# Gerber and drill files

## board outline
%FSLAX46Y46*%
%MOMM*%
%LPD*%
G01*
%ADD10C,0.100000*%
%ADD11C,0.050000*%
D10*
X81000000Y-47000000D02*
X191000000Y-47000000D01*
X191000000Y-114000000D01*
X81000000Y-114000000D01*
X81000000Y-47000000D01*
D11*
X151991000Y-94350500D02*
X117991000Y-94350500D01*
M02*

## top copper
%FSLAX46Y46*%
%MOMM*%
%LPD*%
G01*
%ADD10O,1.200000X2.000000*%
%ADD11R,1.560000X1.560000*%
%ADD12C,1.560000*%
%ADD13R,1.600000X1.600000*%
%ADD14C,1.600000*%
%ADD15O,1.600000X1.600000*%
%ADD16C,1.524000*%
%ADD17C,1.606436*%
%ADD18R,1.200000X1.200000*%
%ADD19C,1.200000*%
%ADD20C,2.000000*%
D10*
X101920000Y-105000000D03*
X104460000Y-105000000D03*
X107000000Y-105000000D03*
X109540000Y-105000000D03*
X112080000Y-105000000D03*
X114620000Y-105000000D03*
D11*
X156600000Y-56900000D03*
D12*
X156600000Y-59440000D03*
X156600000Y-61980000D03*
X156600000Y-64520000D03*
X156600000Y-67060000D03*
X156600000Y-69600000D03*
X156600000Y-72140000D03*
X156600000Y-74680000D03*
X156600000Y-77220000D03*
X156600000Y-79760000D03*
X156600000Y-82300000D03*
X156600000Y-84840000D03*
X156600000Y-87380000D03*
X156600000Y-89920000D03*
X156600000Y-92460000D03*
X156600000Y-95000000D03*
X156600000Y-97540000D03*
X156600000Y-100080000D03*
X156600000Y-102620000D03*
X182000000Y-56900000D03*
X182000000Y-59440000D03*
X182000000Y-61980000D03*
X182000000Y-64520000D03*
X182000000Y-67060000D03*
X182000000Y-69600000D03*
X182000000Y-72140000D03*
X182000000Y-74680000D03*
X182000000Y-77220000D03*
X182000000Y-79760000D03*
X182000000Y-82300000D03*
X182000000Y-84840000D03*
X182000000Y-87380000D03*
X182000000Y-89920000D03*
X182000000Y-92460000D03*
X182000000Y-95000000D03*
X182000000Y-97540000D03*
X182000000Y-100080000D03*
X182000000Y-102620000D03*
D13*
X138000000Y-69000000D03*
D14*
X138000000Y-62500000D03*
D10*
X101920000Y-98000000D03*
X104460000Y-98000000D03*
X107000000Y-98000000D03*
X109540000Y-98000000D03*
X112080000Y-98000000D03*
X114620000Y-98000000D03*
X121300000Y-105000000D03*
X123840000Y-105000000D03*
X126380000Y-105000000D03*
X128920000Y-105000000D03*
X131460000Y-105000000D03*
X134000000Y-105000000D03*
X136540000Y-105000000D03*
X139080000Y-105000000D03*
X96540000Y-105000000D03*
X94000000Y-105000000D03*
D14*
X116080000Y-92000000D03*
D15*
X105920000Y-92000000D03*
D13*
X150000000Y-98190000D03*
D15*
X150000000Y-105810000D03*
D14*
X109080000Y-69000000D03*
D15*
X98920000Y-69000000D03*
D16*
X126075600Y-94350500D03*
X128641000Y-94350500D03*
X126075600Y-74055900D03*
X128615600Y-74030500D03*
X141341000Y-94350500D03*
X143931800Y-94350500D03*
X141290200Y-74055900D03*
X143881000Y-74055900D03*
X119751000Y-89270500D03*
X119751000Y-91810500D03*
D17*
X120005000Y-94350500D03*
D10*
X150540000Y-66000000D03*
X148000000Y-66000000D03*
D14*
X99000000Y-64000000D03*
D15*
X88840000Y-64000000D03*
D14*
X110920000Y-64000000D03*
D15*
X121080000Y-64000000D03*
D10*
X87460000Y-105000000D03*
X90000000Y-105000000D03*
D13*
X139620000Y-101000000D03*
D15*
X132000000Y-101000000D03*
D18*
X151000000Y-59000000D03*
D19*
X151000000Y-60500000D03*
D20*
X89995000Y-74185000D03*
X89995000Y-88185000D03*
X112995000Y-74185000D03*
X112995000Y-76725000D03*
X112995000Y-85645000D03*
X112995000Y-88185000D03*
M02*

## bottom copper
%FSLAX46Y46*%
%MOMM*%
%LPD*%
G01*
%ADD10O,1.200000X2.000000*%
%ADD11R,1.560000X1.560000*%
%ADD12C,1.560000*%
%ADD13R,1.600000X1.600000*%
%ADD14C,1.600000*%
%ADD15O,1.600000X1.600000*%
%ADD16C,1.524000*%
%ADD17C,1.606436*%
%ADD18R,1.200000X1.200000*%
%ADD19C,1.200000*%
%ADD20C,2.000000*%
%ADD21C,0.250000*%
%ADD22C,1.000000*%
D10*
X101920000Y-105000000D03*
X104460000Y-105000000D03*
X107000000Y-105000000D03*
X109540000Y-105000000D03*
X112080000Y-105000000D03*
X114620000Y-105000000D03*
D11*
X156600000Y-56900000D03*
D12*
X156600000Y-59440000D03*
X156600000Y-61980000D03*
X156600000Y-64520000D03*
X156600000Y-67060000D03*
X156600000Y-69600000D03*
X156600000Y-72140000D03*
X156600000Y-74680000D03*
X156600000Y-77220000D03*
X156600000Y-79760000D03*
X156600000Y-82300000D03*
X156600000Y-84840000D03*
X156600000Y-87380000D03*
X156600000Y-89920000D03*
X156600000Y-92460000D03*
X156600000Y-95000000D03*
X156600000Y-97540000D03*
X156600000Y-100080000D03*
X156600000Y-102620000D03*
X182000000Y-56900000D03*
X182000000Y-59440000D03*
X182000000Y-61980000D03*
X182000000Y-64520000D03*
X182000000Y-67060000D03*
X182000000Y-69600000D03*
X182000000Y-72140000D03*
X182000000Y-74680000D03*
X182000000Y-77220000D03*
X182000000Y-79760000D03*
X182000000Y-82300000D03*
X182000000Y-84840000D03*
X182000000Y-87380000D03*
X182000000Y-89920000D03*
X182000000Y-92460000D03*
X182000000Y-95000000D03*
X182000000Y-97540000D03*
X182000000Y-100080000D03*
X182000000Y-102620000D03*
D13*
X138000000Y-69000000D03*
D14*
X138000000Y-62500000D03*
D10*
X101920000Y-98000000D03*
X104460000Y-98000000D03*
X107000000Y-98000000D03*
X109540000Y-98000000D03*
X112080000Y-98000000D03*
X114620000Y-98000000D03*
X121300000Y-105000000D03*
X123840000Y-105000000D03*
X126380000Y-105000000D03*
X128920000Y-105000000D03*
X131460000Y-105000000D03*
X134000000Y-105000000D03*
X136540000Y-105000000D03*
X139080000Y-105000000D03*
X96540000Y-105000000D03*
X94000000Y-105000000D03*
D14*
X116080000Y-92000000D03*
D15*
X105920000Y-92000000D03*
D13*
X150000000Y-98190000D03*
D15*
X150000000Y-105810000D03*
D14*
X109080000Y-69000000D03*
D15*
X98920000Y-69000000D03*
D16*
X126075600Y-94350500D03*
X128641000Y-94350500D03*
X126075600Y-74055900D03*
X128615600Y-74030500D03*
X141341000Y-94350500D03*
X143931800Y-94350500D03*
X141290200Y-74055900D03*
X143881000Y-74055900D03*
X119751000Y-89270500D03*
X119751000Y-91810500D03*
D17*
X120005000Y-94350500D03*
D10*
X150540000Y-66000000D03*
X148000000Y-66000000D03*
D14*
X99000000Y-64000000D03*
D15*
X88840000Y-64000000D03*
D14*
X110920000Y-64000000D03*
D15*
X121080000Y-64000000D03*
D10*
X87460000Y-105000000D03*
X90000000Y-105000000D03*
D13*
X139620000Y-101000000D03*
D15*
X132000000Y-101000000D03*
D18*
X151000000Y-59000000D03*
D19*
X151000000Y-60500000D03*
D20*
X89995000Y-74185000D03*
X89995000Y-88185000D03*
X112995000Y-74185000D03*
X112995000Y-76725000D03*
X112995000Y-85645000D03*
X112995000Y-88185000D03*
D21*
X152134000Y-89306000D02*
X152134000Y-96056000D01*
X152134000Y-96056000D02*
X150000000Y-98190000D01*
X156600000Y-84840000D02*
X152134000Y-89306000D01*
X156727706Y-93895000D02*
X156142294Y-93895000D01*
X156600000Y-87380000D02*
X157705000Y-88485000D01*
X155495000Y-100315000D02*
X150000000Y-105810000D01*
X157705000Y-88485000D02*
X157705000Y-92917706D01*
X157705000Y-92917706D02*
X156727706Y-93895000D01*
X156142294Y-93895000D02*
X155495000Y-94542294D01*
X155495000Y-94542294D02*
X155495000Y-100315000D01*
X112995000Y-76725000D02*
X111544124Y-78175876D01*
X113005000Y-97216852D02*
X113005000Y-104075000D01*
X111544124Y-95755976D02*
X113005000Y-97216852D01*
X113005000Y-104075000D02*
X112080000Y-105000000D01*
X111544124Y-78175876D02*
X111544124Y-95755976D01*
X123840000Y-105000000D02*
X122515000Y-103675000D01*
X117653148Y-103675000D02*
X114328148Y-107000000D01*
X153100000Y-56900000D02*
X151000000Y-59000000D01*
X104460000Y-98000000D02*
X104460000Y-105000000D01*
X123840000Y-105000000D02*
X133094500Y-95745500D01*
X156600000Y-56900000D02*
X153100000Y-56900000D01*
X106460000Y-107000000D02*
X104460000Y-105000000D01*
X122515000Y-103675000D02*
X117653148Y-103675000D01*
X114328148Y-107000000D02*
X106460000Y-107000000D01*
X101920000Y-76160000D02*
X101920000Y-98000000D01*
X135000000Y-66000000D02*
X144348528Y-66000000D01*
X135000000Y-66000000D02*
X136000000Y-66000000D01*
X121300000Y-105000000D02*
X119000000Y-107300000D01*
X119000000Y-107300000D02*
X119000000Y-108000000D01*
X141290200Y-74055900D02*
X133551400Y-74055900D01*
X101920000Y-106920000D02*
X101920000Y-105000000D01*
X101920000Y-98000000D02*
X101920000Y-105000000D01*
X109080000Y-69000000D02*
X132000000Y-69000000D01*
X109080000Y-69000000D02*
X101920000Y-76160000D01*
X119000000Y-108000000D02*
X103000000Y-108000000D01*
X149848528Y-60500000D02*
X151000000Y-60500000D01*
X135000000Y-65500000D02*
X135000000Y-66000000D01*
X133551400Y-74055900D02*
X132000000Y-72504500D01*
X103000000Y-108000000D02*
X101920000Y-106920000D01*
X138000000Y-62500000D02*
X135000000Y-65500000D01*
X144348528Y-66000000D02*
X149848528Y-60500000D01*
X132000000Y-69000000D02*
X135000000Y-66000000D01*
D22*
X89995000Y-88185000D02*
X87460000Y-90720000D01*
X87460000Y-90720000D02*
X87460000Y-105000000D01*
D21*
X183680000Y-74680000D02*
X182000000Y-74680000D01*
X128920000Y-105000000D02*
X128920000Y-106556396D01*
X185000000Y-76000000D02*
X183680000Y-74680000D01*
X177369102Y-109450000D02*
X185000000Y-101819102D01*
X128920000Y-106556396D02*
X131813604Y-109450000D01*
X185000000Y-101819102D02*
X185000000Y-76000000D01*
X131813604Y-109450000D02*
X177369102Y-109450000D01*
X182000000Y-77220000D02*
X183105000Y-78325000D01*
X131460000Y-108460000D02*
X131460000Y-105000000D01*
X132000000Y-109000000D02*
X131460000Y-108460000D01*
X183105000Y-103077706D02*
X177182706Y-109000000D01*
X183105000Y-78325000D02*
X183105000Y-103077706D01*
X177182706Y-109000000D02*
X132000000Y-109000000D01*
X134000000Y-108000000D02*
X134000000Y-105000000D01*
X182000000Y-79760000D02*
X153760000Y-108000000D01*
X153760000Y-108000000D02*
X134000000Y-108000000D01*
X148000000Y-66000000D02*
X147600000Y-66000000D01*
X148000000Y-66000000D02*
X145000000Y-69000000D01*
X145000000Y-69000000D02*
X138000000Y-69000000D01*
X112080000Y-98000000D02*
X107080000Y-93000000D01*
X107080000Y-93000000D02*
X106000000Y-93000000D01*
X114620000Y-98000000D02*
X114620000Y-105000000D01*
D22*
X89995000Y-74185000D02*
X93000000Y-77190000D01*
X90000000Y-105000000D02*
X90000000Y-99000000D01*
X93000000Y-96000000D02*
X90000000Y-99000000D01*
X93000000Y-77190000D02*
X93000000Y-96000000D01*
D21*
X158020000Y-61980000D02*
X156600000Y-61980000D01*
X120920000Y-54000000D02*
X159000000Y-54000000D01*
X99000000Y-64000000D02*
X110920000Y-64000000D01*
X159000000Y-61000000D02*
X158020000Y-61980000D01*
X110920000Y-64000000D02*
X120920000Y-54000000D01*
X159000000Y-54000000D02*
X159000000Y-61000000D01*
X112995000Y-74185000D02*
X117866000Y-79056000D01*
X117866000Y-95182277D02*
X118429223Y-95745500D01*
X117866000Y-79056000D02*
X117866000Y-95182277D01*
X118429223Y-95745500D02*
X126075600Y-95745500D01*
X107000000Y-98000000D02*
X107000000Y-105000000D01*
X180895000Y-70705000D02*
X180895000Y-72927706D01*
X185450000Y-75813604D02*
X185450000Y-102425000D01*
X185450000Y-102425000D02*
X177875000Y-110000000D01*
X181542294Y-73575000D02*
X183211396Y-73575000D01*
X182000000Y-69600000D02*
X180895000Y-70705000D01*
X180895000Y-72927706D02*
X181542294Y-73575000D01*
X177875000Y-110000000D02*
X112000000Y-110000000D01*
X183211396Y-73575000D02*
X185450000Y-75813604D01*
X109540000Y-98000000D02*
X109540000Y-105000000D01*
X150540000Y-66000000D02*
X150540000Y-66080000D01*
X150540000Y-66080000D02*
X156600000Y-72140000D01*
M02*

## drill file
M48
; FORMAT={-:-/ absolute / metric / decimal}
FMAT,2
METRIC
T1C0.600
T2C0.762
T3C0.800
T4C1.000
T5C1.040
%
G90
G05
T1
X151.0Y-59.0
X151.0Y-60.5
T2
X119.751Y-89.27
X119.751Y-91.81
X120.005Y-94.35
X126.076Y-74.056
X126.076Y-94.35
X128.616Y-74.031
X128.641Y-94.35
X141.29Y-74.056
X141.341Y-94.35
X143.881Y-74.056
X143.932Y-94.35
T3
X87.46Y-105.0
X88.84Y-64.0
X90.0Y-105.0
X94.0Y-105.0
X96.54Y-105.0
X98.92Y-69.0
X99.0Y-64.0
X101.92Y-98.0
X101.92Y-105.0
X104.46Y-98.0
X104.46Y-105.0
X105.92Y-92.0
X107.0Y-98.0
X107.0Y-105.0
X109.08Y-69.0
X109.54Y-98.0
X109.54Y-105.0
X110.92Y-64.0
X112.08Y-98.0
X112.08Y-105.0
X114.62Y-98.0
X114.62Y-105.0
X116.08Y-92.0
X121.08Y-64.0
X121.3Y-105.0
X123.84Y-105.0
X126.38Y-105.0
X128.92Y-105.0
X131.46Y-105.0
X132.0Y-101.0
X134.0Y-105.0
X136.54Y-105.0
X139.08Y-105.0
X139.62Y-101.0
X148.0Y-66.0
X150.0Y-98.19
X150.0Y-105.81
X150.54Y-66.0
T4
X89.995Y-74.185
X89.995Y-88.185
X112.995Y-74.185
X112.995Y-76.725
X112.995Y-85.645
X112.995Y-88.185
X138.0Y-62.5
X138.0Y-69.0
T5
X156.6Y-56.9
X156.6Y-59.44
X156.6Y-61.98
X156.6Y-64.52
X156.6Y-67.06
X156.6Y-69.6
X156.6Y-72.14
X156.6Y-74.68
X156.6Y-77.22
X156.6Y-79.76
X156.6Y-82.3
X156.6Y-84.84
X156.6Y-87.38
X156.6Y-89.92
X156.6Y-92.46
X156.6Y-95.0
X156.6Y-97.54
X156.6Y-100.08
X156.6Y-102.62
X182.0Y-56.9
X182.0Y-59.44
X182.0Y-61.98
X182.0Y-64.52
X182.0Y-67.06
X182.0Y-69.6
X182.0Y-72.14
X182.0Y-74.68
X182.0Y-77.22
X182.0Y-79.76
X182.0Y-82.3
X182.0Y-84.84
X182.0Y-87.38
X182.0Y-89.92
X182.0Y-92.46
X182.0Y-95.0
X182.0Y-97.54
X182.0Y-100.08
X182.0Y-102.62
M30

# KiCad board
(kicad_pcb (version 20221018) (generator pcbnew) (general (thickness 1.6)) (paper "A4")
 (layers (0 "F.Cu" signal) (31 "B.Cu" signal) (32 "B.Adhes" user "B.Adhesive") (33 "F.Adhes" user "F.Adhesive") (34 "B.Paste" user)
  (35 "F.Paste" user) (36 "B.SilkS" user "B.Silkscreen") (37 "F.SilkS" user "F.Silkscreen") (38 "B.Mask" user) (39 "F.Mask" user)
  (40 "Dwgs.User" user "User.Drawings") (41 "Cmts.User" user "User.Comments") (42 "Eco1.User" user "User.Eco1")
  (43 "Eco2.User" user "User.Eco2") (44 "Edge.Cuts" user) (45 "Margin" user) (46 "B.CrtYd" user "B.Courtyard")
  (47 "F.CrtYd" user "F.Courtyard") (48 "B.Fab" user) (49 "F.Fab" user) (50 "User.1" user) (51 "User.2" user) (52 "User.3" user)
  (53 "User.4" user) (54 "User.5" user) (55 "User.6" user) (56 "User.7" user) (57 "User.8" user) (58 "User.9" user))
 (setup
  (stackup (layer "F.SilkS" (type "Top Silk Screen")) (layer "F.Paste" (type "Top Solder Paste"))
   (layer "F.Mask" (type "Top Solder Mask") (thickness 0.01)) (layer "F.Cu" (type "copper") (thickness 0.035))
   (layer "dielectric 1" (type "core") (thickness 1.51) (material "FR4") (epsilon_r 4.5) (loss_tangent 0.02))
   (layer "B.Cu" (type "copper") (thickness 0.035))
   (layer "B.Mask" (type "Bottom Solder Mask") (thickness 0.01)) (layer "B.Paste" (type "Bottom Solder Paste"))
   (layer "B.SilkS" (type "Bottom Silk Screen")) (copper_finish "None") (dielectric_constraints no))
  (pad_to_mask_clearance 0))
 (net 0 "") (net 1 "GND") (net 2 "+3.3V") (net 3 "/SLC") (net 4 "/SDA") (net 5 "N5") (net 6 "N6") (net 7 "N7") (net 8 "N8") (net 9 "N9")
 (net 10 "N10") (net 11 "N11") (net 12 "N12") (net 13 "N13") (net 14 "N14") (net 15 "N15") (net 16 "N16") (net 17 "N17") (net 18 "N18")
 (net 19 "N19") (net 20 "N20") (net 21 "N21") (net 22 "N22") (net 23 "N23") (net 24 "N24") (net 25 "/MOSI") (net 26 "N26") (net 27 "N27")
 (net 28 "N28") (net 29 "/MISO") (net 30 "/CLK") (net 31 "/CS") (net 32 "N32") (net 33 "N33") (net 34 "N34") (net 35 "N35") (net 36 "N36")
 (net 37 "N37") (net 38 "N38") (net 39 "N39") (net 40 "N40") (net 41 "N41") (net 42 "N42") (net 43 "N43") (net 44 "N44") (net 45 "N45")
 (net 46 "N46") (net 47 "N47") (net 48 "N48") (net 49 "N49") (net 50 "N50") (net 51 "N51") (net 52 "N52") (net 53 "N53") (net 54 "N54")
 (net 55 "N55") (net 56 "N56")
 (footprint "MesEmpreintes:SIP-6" (layer "F.Cu") (at 108.27 105)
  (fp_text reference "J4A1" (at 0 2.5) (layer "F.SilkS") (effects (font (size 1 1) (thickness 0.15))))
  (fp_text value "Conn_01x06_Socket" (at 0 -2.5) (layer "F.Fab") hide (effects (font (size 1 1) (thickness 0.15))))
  (pad "1" thru_hole oval (at -6.35 0) (size 1.2 2) (drill 0.8) (layers "*.Cu" "*.Mask") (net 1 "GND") (thermal_bridge_angle 45))
  (pad "2" thru_hole oval (at -3.81 0) (size 1.2 2) (drill 0.8) (layers "*.Cu" "*.Mask") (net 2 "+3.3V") (thermal_bridge_angle 45))
  (pad "3" thru_hole oval (at -1.27 0) (size 1.2 2) (drill 0.8) (layers "*.Cu" "*.Mask") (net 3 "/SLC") (thermal_bridge_angle 45))
  (pad "4" thru_hole oval (at 1.27 0) (size 1.2 2) (drill 0.8) (layers "*.Cu" "*.Mask") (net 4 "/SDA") (thermal_bridge_angle 45))
  (pad "5" thru_hole oval (at 3.81 0) (size 1.2 2) (drill 0.8) (layers "*.Cu" "*.Mask") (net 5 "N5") (thermal_bridge_angle 45))
  (pad "6" thru_hole oval (at 6.35 0) (size 1.2 2) (drill 0.8) (layers "*.Cu" "*.Mask") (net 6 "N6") (thermal_bridge_angle 45)))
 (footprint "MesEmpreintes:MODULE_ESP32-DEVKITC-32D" (layer "F.Cu") (at 169.3 75.97)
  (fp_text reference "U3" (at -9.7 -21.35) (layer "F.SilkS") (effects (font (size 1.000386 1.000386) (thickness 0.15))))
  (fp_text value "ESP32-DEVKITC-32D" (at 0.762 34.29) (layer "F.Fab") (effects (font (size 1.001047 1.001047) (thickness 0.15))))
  (pad "J2-1" thru_hole rect (at -12.7 -19.07) (size 1.56 1.56) (drill 1.04) (layers "*.Cu" "*.Mask") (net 2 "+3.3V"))
  (pad "J2-2" thru_hole circle (at -12.7 -16.53) (size 1.56 1.56) (drill 1.04) (layers "*.Cu" "*.Mask") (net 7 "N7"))
  (pad "J2-3" thru_hole circle (at -12.7 -13.99) (size 1.56 1.56) (drill 1.04) (layers "*.Cu" "*.Mask") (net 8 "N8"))
  (pad "J2-4" thru_hole circle (at -12.7 -11.45) (size 1.56 1.56) (drill 1.04) (layers "*.Cu" "*.Mask") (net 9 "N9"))
  (pad "J2-5" thru_hole circle (at -12.7 -8.91) (size 1.56 1.56) (drill 1.04) (layers "*.Cu" "*.Mask") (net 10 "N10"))
  (pad "J2-6" thru_hole circle (at -12.7 -6.37) (size 1.56 1.56) (drill 1.04) (layers "*.Cu" "*.Mask") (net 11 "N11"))
  (pad "J2-7" thru_hole circle (at -12.7 -3.83) (size 1.56 1.56) (drill 1.04) (layers "*.Cu" "*.Mask") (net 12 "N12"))
  (pad "J2-8" thru_hole circle (at -12.7 -1.29) (size 1.56 1.56) (drill 1.04) (layers "*.Cu" "*.Mask") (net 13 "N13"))
  (pad "J2-9" thru_hole circle (at -12.7 1.25) (size 1.56 1.56) (drill 1.04) (layers "*.Cu" "*.Mask") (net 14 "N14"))
  (pad "J2-10" thru_hole circle (at -12.7 3.79) (size 1.56 1.56) (drill 1.04) (layers "*.Cu" "*.Mask") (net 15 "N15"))
  (pad "J2-11" thru_hole circle (at -12.7 6.33) (size 1.56 1.56) (drill 1.04) (layers "*.Cu" "*.Mask") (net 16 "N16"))
  (pad "J2-12" thru_hole circle (at -12.7 8.87) (size 1.56 1.56) (drill 1.04) (layers "*.Cu" "*.Mask") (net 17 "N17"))
  (pad "J2-13" thru_hole circle (at -12.7 11.41) (size 1.56 1.56) (drill 1.04) (layers "*.Cu" "*.Mask") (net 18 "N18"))
  (pad "J2-14" thru_hole circle (at -12.7 13.95) (size 1.56 1.56) (drill 1.04) (layers "*.Cu" "*.Mask") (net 1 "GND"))
  (pad "J2-15" thru_hole circle (at -12.7 16.49) (size 1.56 1.56) (drill 1.04) (layers "*.Cu" "*.Mask") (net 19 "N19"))
  (pad "J2-16" thru_hole circle (at -12.7 19.03) (size 1.56 1.56) (drill 1.04) (layers "*.Cu" "*.Mask") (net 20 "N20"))
  (pad "J2-17" thru_hole circle (at -12.7 21.57) (size 1.56 1.56) (drill 1.04) (layers "*.Cu" "*.Mask") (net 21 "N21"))
  (pad "J2-18" thru_hole circle (at -12.7 24.11) (size 1.56 1.56) (drill 1.04) (layers "*.Cu" "*.Mask") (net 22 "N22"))
  (pad "J2-19" thru_hole circle (at -12.7 26.65) (size 1.56 1.56) (drill 1.04) (layers "*.Cu" "*.Mask") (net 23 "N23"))
  (pad "J3-1" thru_hole circle (at 12.7 -19.07) (size 1.56 1.56) (drill 1.04) (layers "*.Cu" "*.Mask") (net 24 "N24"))
  (pad "J3-2" thru_hole circle (at 12.7 -16.53) (size 1.56 1.56) (drill 1.04) (layers "*.Cu" "*.Mask") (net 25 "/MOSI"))
  (pad "J3-3" thru_hole circle (at 12.7 -13.99) (size 1.56 1.56) (drill 1.04) (layers "*.Cu" "*.Mask") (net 3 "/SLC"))
  (pad "J3-4" thru_hole circle (at 12.7 -11.45) (size 1.56 1.56) (drill 1.04) (layers "*.Cu" "*.Mask") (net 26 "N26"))
  (pad "J3-5" thru_hole circle (at 12.7 -8.91) (size 1.56 1.56) (drill 1.04) (layers "*.Cu" "*.Mask") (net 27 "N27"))
  (pad "J3-6" thru_hole circle (at 12.7 -6.37) (size 1.56 1.56) (drill 1.04) (layers "*.Cu" "*.Mask") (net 4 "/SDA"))
  (pad "J3-7" thru_hole circle (at 12.7 -3.83) (size 1.56 1.56) (drill 1.04) (layers "*.Cu" "*.Mask") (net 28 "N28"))
  (pad "J3-8" thru_hole circle (at 12.7 -1.29) (size 1.56 1.56) (drill 1.04) (layers "*.Cu" "*.Mask") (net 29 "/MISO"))
  (pad "J3-9" thru_hole circle (at 12.7 1.25) (size 1.56 1.56) (drill 1.04) (layers "*.Cu" "*.Mask") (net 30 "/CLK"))
  (pad "J3-10" thru_hole circle (at 12.7 3.79) (size 1.56 1.56) (drill 1.04) (layers "*.Cu" "*.Mask") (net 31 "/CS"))
  (pad "J3-11" thru_hole circle (at 12.7 6.33) (size 1.56 1.56) (drill 1.04) (layers "*.Cu" "*.Mask") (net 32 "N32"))
  (pad "J3-12" thru_hole circle (at 12.7 8.87) (size 1.56 1.56) (drill 1.04) (layers "*.Cu" "*.Mask") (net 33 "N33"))
  (pad "J3-13" thru_hole circle (at 12.7 11.41) (size 1.56 1.56) (drill 1.04) (layers "*.Cu" "*.Mask") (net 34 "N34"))
  (pad "J3-14" thru_hole circle (at 12.7 13.95) (size 1.56 1.56) (drill 1.04) (layers "*.Cu" "*.Mask") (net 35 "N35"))
  (pad "J3-15" thru_hole circle (at 12.7 16.49) (size 1.56 1.56) (drill 1.04) (layers "*.Cu" "*.Mask") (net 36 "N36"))
  (pad "J3-16" thru_hole circle (at 12.7 19.03) (size 1.56 1.56) (drill 1.04) (layers "*.Cu" "*.Mask") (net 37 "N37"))
  (pad "J3-17" thru_hole circle (at 12.7 21.57) (size 1.56 1.56) (drill 1.04) (layers "*.Cu" "*.Mask") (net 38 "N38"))
  (pad "J3-18" thru_hole circle (at 12.7 24.11) (size 1.56 1.56) (drill 1.04) (layers "*.Cu" "*.Mask") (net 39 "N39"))
  (pad "J3-19" thru_hole circle (at 12.7 26.65) (size 1.56 1.56) (drill 1.04) (layers "*.Cu" "*.Mask") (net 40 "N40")))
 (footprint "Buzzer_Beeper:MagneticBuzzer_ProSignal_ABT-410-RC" (layer "F.Cu") (at 138 69 90)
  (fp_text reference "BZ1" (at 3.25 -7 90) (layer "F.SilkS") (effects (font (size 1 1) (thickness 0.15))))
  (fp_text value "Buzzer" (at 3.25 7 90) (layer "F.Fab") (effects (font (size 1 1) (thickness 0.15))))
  (pad "1" thru_hole rect (at 0 0 90) (size 1.6 1.6) (drill 1) (layers "*.Cu" "*.Mask") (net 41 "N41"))
  (pad "2" thru_hole circle (at 6.5 0 90) (size 1.6 1.6) (drill 1) (layers "*.Cu" "*.Mask") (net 1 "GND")))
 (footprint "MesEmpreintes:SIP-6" (layer "F.Cu") (at 108.27 98)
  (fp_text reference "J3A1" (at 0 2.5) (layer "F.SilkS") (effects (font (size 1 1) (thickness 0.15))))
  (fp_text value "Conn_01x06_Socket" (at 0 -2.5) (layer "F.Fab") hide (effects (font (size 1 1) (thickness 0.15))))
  (pad "1" thru_hole oval (at -6.35 0) (size 1.2 2) (drill 0.8) (layers "*.Cu" "*.Mask") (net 1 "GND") (thermal_bridge_angle 45))
  (pad "2" thru_hole oval (at -3.81 0) (size 1.2 2) (drill 0.8) (layers "*.Cu" "*.Mask") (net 2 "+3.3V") (thermal_bridge_angle 45))
  (pad "3" thru_hole oval (at -1.27 0) (size 1.2 2) (drill 0.8) (layers "*.Cu" "*.Mask") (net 3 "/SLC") (thermal_bridge_angle 45))
  (pad "4" thru_hole oval (at 1.27 0) (size 1.2 2) (drill 0.8) (layers "*.Cu" "*.Mask") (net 4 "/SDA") (thermal_bridge_angle 45))
  (pad "5" thru_hole oval (at 3.81 0) (size 1.2 2) (drill 0.8) (layers "*.Cu" "*.Mask") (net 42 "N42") (thermal_bridge_angle 45))
  (pad "6" thru_hole oval (at 6.35 0) (size 1.2 2) (drill 0.8) (layers "*.Cu" "*.Mask") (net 6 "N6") (thermal_bridge_angle 45)))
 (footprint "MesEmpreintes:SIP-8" (layer "F.Cu") (at 130.19 105)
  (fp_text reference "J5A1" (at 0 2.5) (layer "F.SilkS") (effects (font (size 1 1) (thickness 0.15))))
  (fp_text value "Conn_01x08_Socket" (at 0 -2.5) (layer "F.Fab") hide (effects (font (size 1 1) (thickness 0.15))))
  (pad "1" thru_hole oval (at -8.89 0) (size 1.2 2) (drill 0.8) (layers "*.Cu" "*.Mask") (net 1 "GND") (thermal_bridge_angle 45))
  (pad "2" thru_hole oval (at -6.35 0) (size 1.2 2) (drill 0.8) (layers "*.Cu" "*.Mask") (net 2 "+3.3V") (thermal_bridge_angle 45))
  (pad "3" thru_hole oval (at -3.81 0) (size 1.2 2) (drill 0.8) (layers "*.Cu" "*.Mask") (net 25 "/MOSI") (thermal_bridge_angle 45))
  (pad "4" thru_hole oval (at -1.27 0) (size 1.2 2) (drill 0.8) (layers "*.Cu" "*.Mask") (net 29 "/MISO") (thermal_bridge_angle 45))
  (pad "5" thru_hole oval (at 1.27 0) (size 1.2 2) (drill 0.8) (layers "*.Cu" "*.Mask") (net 30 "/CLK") (thermal_bridge_angle 45))
  (pad "6" thru_hole oval (at 3.81 0) (size 1.2 2) (drill 0.8) (layers "*.Cu" "*.Mask") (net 31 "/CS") (thermal_bridge_angle 45))
  (pad "7" thru_hole oval (at 6.35 0) (size 1.2 2) (drill 0.8) (layers "*.Cu" "*.Mask") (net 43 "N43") (thermal_bridge_angle 45))
  (pad "8" thru_hole oval (at 8.89 0) (size 1.2 2) (drill 0.8) (layers "*.Cu" "*.Mask") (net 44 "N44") (thermal_bridge_angle 45)))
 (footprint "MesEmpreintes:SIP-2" (layer "F.Cu") (at 95.27 105 180)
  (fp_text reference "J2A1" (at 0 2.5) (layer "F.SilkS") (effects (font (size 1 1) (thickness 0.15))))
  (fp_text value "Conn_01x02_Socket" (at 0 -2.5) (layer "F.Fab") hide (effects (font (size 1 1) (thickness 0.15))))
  (pad "1" thru_hole oval (at -1.27 0 180) (size 1.2 2) (drill 0.8) (layers "*.Cu" "*.Mask") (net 6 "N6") (thermal_bridge_angle 45))
  (pad "2" thru_hole oval (at 1.27 0 180) (size 1.2 2) (drill 0.8) (layers "*.Cu" "*.Mask") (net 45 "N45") (thermal_bridge_angle 45)))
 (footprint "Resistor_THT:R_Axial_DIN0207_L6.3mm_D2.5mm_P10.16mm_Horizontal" (layer "F.Cu") (at 116.08 92 180)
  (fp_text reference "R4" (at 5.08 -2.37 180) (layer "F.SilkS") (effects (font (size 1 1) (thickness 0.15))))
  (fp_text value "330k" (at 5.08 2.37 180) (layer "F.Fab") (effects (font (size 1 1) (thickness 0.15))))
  (pad "1" thru_hole circle (at 0 0 180) (size 1.6 1.6) (drill 0.8) (layers "*.Cu" "*.Mask") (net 42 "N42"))
  (pad "2" thru_hole oval (at 10.16 0 180) (size 1.6 1.6) (drill 0.8) (layers "*.Cu" "*.Mask") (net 17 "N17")))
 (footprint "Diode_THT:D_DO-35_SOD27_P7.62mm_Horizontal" (layer "F.Cu") (at 150 98.19 -90)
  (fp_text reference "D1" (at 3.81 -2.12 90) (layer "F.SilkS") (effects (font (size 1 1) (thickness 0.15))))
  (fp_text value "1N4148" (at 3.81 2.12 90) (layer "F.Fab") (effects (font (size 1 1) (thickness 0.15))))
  (pad "1" thru_hole rect (at 0 0 270) (size 1.6 1.6) (drill 0.8) (layers "*.Cu" "*.Mask") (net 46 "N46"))
  (pad "2" thru_hole oval (at 7.62 0 270) (size 1.6 1.6) (drill 0.8) (layers "*.Cu" "*.Mask") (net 18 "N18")))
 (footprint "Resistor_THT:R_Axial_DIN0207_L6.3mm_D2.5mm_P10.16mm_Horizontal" (layer "F.Cu") (at 109.08 69 180)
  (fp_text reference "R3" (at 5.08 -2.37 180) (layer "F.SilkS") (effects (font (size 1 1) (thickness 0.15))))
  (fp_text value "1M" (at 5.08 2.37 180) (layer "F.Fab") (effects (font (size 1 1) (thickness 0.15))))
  (pad "1" thru_hole circle (at 0 0 180) (size 1.6 1.6) (drill 0.8) (layers "*.Cu" "*.Mask") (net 1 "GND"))
  (pad "2" thru_hole oval (at 10.16 0 180) (size 1.6 1.6) (drill 0.8) (layers "*.Cu" "*.Mask") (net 46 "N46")))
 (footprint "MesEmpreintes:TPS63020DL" (layer "F.Cu") (at 134.991 94.3505 90)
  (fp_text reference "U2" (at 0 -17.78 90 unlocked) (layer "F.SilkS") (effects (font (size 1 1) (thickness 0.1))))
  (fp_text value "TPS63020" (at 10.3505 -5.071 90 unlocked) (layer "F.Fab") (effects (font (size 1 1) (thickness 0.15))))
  (fp_line (start 0 17) (end 0 -17) (stroke (width 0.05) (type default)) (layer "Edge.Cuts"))
  (pad "1" thru_hole circle (at 0 -8.9154 90) (size 1.524 1.524) (drill 0.762) (layers "*.Cu" "*.Mask") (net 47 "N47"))
  (pad "2" thru_hole circle (at 0 -6.35 90) (size 1.524 1.524) (drill 0.762) (layers "*.Cu" "*.Mask") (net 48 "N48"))
  (pad "3" thru_hole circle (at 20.2946 -8.9154 90) (size 1.524 1.524) (drill 0.762) (layers "*.Cu" "*.Mask") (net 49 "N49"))
  (pad "4" thru_hole circle (at 20.32 -6.3754 90) (size 1.524 1.524) (drill 0.762) (layers "*.Cu" "*.Mask") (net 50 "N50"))
  (pad "5" thru_hole circle (at 0 6.35 90) (size 1.524 1.524) (drill 0.762) (layers "*.Cu" "*.Mask") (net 2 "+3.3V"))
  (pad "6" thru_hole circle (at 0 8.9408 90) (size 1.524 1.524) (drill 0.762) (layers "*.Cu" "*.Mask") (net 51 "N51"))
  (pad "7" thru_hole circle (at 20.2946 6.2992 90) (size 1.524 1.524) (drill 0.762) (layers "*.Cu" "*.Mask") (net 1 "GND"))
  (pad "8" thru_hole circle (at 20.2946 8.89 90) (size 1.524 1.524) (drill 0.762) (layers "*.Cu" "*.Mask") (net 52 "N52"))
  (pad "9" thru_hole circle (at 5.08 -15.24 90) (size 1.524 1.524) (drill 0.762) (layers "*.Cu" "*.Mask") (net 46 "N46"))
  (pad "10" thru_hole circle (at 2.54 -15.24 90) (size 1.524 1.524) (drill 0.762) (layers "*.Cu" "*.Mask") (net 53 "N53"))
  (pad "11" thru_hole circle (at 0 -14.986 90) (size 1.606436 1.606436) (drill 0.762) (layers "*.Cu" "*.Mask") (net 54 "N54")))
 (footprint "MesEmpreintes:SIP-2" (layer "F.Cu") (at 149.27 66 180)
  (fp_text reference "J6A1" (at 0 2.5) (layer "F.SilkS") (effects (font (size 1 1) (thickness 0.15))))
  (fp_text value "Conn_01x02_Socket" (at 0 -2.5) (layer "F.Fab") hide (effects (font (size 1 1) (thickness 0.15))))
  (pad "1" thru_hole oval (at -1.27 0 180) (size 1.2 2) (drill 0.8) (layers "*.Cu" "*.Mask") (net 12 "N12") (thermal_bridge_angle 45))
  (pad "2" thru_hole oval (at 1.27 0 180) (size 1.2 2) (drill 0.8) (layers "*.Cu" "*.Mask") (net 41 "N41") (thermal_bridge_angle 45)))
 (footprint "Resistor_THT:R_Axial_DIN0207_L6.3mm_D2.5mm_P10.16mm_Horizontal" (layer "F.Cu") (at 99 64 180)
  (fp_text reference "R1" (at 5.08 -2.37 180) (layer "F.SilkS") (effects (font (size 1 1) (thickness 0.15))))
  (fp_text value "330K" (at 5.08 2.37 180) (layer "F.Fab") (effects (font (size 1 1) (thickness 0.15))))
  (pad "1" thru_hole circle (at 0 0 180) (size 1.6 1.6) (drill 0.8) (layers "*.Cu" "*.Mask") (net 8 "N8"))
  (pad "2" thru_hole oval (at 10.16 0 180) (size 1.6 1.6) (drill 0.8) (layers "*.Cu" "*.Mask") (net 45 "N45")))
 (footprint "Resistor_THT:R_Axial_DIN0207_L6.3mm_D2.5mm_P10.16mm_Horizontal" (layer "F.Cu") (at 110.92 64)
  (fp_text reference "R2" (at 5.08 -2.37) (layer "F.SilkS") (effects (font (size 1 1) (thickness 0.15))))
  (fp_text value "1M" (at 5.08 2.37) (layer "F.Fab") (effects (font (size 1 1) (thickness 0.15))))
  (pad "1" thru_hole circle (at 0 0) (size 1.6 1.6) (drill 0.8) (layers "*.Cu" "*.Mask") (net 8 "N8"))
  (pad "2" thru_hole oval (at 10.16 0) (size 1.6 1.6) (drill 0.8) (layers "*.Cu" "*.Mask") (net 5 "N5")))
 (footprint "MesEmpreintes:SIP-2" (layer "F.Cu") (at 88.73 105)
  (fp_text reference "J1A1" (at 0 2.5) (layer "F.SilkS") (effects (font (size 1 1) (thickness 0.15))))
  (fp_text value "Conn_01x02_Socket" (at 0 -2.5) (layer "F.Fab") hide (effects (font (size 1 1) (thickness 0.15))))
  (pad "1" thru_hole oval (at -1.27 0) (size 1.2 2) (drill 0.8) (layers "*.Cu" "*.Mask") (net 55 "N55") (thermal_bridge_angle 45))
  (pad "2" thru_hole oval (at 1.27 0) (size 1.2 2) (drill 0.8) (layers "*.Cu" "*.Mask") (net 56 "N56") (thermal_bridge_angle 45)))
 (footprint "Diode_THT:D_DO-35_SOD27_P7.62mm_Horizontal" (layer "F.Cu") (at 139.62 101 180)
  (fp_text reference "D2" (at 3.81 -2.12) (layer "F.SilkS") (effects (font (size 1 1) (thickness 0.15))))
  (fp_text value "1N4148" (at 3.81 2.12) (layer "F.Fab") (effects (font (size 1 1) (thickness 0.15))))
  (pad "1" thru_hole rect (at 0 0 180) (size 1.6 1.6) (drill 0.8) (layers "*.Cu" "*.Mask") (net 46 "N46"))
  (pad "2" thru_hole oval (at 7.62 0 180) (size 1.6 1.6) (drill 0.8) (layers "*.Cu" "*.Mask") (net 17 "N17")))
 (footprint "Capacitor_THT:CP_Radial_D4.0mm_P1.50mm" (layer "F.Cu") (at 151 59 -90)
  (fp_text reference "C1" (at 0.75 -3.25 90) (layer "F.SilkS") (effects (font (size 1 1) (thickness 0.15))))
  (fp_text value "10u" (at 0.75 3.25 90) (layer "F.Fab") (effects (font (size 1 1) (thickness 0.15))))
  (pad "1" thru_hole rect (at 0 0 270) (size 1.2 1.2) (drill 0.6) (layers "*.Cu" "*.Mask") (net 2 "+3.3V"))
  (pad "2" thru_hole circle (at 1.5 0 270) (size 1.2 1.2) (drill 0.6) (layers "*.Cu" "*.Mask") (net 1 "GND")))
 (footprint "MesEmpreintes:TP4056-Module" (layer "F.Cu") (at 87.495 89.785)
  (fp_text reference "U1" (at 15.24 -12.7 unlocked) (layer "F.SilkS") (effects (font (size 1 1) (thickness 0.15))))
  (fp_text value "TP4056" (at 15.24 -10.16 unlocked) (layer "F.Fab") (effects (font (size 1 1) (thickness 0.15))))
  (pad "1" thru_hole circle (at 2.5 -15.6) (size 2 2) (drill 1) (layers "*.Cu" "*.Mask") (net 56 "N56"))
  (pad "2" thru_hole circle (at 2.5 -1.6) (size 2 2) (drill 1) (layers "*.Cu" "*.Mask") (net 55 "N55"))
  (pad "3" thru_hole circle (at 25.5 -15.6) (size 2 2) (drill 1) (layers "*.Cu" "*.Mask") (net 47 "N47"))
  (pad "4" thru_hole circle (at 25.5 -13.06) (size 2 2) (drill 1) (layers "*.Cu" "*.Mask") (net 5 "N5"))
  (pad "5" thru_hole circle (at 25.5 -4.14) (size 2 2) (drill 1) (layers "*.Cu" "*.Mask") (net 45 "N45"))
  (pad "6" thru_hole circle (at 25.5 -1.6) (size 2 2) (drill 1) (layers "*.Cu" "*.Mask") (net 49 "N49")))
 (gr_rect (start 81 47) (end 191 114) (stroke (width 0.1) (type default)) (fill none) (layer "Edge.Cuts"))
 (segment (start 152.134 89.306) (end 152.134 96.056) (width 0.25) (layer "B.Cu") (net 46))
 (segment (start 152.134 96.056) (end 150 98.19) (width 0.25) (layer "B.Cu") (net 46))
 (segment (start 156.6 84.84) (end 152.134 89.306) (width 0.25) (layer "B.Cu") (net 46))
 (segment (start 156.727706 93.895) (end 156.142294 93.895) (width 0.25) (layer "B.Cu") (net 18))
 (segment (start 156.6 87.38) (end 157.705 88.485) (width 0.25) (layer "B.Cu") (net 18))
 (segment (start 155.495 100.315) (end 150 105.81) (width 0.25) (layer "B.Cu") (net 18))
 (segment (start 157.705 88.485) (end 157.705 92.917706) (width 0.25) (layer "B.Cu") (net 18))
 (segment (start 157.705 92.917706) (end 156.727706 93.895) (width 0.25) (layer "B.Cu") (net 18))
 (segment (start 156.142294 93.895) (end 155.495 94.542294) (width 0.25) (layer "B.Cu") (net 18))
 (segment (start 155.495 94.542294) (end 155.495 100.315) (width 0.25) (layer "B.Cu") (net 18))
 (segment (start 112.995 76.725) (end 111.544124 78.175876) (width 0.25) (layer "B.Cu") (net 5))
 (segment (start 113.005 97.216852) (end 113.005 104.075) (width 0.25) (layer "B.Cu") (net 5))
 (segment (start 111.544124 95.755976) (end 113.005 97.216852) (width 0.25) (layer "B.Cu") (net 5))
 (segment (start 113.005 104.075) (end 112.08 105) (width 0.25) (layer "B.Cu") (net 5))
 (segment (start 111.544124 78.175876) (end 111.544124 95.755976) (width 0.25) (layer "B.Cu") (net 5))
 (segment (start 123.84 105) (end 122.515 103.675) (width 0.25) (layer "B.Cu") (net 2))
 (segment (start 117.653148 103.675) (end 114.328148 107) (width 0.25) (layer "B.Cu") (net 2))
 (segment (start 153.1 56.9) (end 151 59) (width 0.25) (layer "B.Cu") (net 2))
 (segment (start 104.46 98) (end 104.46 105) (width 0.25) (layer "B.Cu") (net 2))
 (segment (start 123.84 105) (end 133.0945 95.7455) (width 0.25) (layer "B.Cu") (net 2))
 (segment (start 156.6 56.9) (end 153.1 56.9) (width 0.25) (layer "B.Cu") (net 2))
 (segment (start 106.46 107) (end 104.46 105) (width 0.25) (layer "B.Cu") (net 2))
 (segment (start 122.515 103.675) (end 117.653148 103.675) (width 0.25) (layer "B.Cu") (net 2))
 (segment (start 114.328148 107) (end 106.46 107) (width 0.25) (layer "B.Cu") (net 2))
 (segment (start 101.92 76.16) (end 101.92 98) (width 0.25) (layer "B.Cu") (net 1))
 (segment (start 135 66) (end 144.348528 66) (width 0.25) (layer "B.Cu") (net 1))
 (segment (start 135 66) (end 136 66) (width 0.25) (layer "B.Cu") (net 1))
 (segment (start 121.3 105) (end 119 107.3) (width 0.25) (layer "B.Cu") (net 1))
 (segment (start 119 107.3) (end 119 108) (width 0.25) (layer "B.Cu") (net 1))
 (segment (start 141.2902 74.0559) (end 133.5514 74.0559) (width 0.25) (layer "B.Cu") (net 1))
 (segment (start 101.92 106.92) (end 101.92 105) (width 0.25) (layer "B.Cu") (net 1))
 (segment (start 101.92 98) (end 101.92 105) (width 0.25) (layer "B.Cu") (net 1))
 (segment (start 109.08 69) (end 132 69) (width 0.25) (layer "B.Cu") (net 1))
 (segment (start 109.08 69) (end 101.92 76.16) (width 0.25) (layer "B.Cu") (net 1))
 (segment (start 119 108) (end 103 108) (width 0.25) (layer "B.Cu") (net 1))
 (segment (start 149.848528 60.5) (end 151 60.5) (width 0.25) (layer "B.Cu") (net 1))
 (segment (start 135 65.5) (end 135 66) (width 0.25) (layer "B.Cu") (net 1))
 (segment (start 133.5514 74.0559) (end 132 72.5045) (width 0.25) (layer "B.Cu") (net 1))
 (segment (start 103 108) (end 101.92 106.92) (width 0.25) (layer "B.Cu") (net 1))
 (segment (start 138 62.5) (end 135 65.5) (width 0.25) (layer "B.Cu") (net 1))
 (segment (start 144.348528 66) (end 149.848528 60.5) (width 0.25) (layer "B.Cu") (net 1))
 (segment (start 132 69) (end 135 66) (width 0.25) (layer "B.Cu") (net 1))
 (segment (start 89.995 88.185) (end 87.46 90.72) (width 1) (layer "B.Cu") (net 55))
 (segment (start 87.46 90.72) (end 87.46 105) (width 1) (layer "B.Cu") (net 55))
 (segment (start 183.68 74.68) (end 182 74.68) (width 0.25) (layer "B.Cu") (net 29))
 (segment (start 128.92 105) (end 128.92 106.556396) (width 0.25) (layer "B.Cu") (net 29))
 (segment (start 185 76) (end 183.68 74.68) (width 0.25) (layer "B.Cu") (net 29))
 (segment (start 177.369102 109.45) (end 185 101.819102) (width 0.25) (layer "B.Cu") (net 29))
 (segment (start 128.92 106.556396) (end 131.813604 109.45) (width 0.25) (layer "B.Cu") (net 29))
 (segment (start 185 101.819102) (end 185 76) (width 0.25) (layer "B.Cu") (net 29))
 (segment (start 131.813604 109.45) (end 177.369102 109.45) (width 0.25) (layer "B.Cu") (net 29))
 (segment (start 182 77.22) (end 183.105 78.325) (width 0.25) (layer "B.Cu") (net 30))
 (segment (start 131.46 108.46) (end 131.46 105) (width 0.25) (layer "B.Cu") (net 30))
 (segment (start 132 109) (end 131.46 108.46) (width 0.25) (layer "B.Cu") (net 30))
 (segment (start 183.105 103.077706) (end 177.182706 109) (width 0.25) (layer "B.Cu") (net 30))
 (segment (start 183.105 78.325) (end 183.105 103.077706) (width 0.25) (layer "B.Cu") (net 30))
 (segment (start 177.182706 109) (end 132 109) (width 0.25) (layer "B.Cu") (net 30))
 (segment (start 134 108) (end 134 105) (width 0.25) (layer "B.Cu") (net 31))
 (segment (start 182 79.76) (end 153.76 108) (width 0.25) (layer "B.Cu") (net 31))
 (segment (start 153.76 108) (end 134 108) (width 0.25) (layer "B.Cu") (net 31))
 (segment (start 148 66) (end 147.6 66) (width 0.25) (layer "B.Cu") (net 41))
 (segment (start 148 66) (end 145 69) (width 0.25) (layer "B.Cu") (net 41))
 (segment (start 145 69) (end 138 69) (width 0.25) (layer "B.Cu") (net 41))
 (segment (start 112.08 98) (end 107.08 93) (width 0.25) (layer "B.Cu") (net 42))
 (segment (start 107.08 93) (end 106 93) (width 0.25) (layer "B.Cu") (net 42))
 (segment (start 114.62 98) (end 114.62 105) (width 0.25) (layer "B.Cu") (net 6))
 (segment (start 89.995 74.185) (end 93 77.19) (width 1) (layer "B.Cu") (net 56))
 (segment (start 90 105) (end 90 99) (width 1) (layer "B.Cu") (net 56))
 (segment (start 93 96) (end 90 99) (width 1) (layer "B.Cu") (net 56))
 (segment (start 93 77.19) (end 93 96) (width 1) (layer "B.Cu") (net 56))
 (segment (start 158.02 61.98) (end 156.6 61.98) (width 0.25) (layer "B.Cu") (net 8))
 (segment (start 120.92 54) (end 159 54) (width 0.25) (layer "B.Cu") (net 8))
 (segment (start 99 64) (end 110.92 64) (width 0.25) (layer "B.Cu") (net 8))
 (segment (start 159 61) (end 158.02 61.98) (width 0.25) (layer "B.Cu") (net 8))
 (segment (start 110.92 64) (end 120.92 54) (width 0.25) (layer "B.Cu") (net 8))
 (segment (start 159 54) (end 159 61) (width 0.25) (layer "B.Cu") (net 8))
 (segment (start 112.995 74.185) (end 117.866 79.056) (width 0.25) (layer "B.Cu") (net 47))
 (segment (start 117.866 95.182277) (end 118.429223 95.7455) (width 0.25) (layer "B.Cu") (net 47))
 (segment (start 117.866 79.056) (end 117.866 95.182277) (width 0.25) (layer "B.Cu") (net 47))
 (segment (start 118.429223 95.7455) (end 126.0756 95.7455) (width 0.25) (layer "B.Cu") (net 47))
 (segment (start 107 98) (end 107 105) (width 0.25) (layer "B.Cu") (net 3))
 (segment (start 180.895 70.705) (end 180.895 72.927706) (width 0.25) (layer "B.Cu") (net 4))
 (segment (start 185.45 75.813604) (end 185.45 102.425) (width 0.25) (layer "B.Cu") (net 4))
 (segment (start 185.45 102.425) (end 177.875 110) (width 0.25) (layer "B.Cu") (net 4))
 (segment (start 181.542294 73.575) (end 183.211396 73.575) (width 0.25) (layer "B.Cu") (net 4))
 (segment (start 182 69.6) (end 180.895 70.705) (width 0.25) (layer "B.Cu") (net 4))
 (segment (start 180.895 72.927706) (end 181.542294 73.575) (width 0.25) (layer "B.Cu") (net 4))
 (segment (start 177.875 110) (end 112 110) (width 0.25) (layer "B.Cu") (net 4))
 (segment (start 183.211396 73.575) (end 185.45 75.813604) (width 0.25) (layer "B.Cu") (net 4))
 (segment (start 109.54 98) (end 109.54 105) (width 0.25) (layer "B.Cu") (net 4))
 (segment (start 150.54 66) (end 150.54 66.08) (width 0.25) (layer "B.Cu") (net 12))
 (segment (start 150.54 66.08) (end 156.6 72.14) (width 0.25) (layer "B.Cu") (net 12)))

